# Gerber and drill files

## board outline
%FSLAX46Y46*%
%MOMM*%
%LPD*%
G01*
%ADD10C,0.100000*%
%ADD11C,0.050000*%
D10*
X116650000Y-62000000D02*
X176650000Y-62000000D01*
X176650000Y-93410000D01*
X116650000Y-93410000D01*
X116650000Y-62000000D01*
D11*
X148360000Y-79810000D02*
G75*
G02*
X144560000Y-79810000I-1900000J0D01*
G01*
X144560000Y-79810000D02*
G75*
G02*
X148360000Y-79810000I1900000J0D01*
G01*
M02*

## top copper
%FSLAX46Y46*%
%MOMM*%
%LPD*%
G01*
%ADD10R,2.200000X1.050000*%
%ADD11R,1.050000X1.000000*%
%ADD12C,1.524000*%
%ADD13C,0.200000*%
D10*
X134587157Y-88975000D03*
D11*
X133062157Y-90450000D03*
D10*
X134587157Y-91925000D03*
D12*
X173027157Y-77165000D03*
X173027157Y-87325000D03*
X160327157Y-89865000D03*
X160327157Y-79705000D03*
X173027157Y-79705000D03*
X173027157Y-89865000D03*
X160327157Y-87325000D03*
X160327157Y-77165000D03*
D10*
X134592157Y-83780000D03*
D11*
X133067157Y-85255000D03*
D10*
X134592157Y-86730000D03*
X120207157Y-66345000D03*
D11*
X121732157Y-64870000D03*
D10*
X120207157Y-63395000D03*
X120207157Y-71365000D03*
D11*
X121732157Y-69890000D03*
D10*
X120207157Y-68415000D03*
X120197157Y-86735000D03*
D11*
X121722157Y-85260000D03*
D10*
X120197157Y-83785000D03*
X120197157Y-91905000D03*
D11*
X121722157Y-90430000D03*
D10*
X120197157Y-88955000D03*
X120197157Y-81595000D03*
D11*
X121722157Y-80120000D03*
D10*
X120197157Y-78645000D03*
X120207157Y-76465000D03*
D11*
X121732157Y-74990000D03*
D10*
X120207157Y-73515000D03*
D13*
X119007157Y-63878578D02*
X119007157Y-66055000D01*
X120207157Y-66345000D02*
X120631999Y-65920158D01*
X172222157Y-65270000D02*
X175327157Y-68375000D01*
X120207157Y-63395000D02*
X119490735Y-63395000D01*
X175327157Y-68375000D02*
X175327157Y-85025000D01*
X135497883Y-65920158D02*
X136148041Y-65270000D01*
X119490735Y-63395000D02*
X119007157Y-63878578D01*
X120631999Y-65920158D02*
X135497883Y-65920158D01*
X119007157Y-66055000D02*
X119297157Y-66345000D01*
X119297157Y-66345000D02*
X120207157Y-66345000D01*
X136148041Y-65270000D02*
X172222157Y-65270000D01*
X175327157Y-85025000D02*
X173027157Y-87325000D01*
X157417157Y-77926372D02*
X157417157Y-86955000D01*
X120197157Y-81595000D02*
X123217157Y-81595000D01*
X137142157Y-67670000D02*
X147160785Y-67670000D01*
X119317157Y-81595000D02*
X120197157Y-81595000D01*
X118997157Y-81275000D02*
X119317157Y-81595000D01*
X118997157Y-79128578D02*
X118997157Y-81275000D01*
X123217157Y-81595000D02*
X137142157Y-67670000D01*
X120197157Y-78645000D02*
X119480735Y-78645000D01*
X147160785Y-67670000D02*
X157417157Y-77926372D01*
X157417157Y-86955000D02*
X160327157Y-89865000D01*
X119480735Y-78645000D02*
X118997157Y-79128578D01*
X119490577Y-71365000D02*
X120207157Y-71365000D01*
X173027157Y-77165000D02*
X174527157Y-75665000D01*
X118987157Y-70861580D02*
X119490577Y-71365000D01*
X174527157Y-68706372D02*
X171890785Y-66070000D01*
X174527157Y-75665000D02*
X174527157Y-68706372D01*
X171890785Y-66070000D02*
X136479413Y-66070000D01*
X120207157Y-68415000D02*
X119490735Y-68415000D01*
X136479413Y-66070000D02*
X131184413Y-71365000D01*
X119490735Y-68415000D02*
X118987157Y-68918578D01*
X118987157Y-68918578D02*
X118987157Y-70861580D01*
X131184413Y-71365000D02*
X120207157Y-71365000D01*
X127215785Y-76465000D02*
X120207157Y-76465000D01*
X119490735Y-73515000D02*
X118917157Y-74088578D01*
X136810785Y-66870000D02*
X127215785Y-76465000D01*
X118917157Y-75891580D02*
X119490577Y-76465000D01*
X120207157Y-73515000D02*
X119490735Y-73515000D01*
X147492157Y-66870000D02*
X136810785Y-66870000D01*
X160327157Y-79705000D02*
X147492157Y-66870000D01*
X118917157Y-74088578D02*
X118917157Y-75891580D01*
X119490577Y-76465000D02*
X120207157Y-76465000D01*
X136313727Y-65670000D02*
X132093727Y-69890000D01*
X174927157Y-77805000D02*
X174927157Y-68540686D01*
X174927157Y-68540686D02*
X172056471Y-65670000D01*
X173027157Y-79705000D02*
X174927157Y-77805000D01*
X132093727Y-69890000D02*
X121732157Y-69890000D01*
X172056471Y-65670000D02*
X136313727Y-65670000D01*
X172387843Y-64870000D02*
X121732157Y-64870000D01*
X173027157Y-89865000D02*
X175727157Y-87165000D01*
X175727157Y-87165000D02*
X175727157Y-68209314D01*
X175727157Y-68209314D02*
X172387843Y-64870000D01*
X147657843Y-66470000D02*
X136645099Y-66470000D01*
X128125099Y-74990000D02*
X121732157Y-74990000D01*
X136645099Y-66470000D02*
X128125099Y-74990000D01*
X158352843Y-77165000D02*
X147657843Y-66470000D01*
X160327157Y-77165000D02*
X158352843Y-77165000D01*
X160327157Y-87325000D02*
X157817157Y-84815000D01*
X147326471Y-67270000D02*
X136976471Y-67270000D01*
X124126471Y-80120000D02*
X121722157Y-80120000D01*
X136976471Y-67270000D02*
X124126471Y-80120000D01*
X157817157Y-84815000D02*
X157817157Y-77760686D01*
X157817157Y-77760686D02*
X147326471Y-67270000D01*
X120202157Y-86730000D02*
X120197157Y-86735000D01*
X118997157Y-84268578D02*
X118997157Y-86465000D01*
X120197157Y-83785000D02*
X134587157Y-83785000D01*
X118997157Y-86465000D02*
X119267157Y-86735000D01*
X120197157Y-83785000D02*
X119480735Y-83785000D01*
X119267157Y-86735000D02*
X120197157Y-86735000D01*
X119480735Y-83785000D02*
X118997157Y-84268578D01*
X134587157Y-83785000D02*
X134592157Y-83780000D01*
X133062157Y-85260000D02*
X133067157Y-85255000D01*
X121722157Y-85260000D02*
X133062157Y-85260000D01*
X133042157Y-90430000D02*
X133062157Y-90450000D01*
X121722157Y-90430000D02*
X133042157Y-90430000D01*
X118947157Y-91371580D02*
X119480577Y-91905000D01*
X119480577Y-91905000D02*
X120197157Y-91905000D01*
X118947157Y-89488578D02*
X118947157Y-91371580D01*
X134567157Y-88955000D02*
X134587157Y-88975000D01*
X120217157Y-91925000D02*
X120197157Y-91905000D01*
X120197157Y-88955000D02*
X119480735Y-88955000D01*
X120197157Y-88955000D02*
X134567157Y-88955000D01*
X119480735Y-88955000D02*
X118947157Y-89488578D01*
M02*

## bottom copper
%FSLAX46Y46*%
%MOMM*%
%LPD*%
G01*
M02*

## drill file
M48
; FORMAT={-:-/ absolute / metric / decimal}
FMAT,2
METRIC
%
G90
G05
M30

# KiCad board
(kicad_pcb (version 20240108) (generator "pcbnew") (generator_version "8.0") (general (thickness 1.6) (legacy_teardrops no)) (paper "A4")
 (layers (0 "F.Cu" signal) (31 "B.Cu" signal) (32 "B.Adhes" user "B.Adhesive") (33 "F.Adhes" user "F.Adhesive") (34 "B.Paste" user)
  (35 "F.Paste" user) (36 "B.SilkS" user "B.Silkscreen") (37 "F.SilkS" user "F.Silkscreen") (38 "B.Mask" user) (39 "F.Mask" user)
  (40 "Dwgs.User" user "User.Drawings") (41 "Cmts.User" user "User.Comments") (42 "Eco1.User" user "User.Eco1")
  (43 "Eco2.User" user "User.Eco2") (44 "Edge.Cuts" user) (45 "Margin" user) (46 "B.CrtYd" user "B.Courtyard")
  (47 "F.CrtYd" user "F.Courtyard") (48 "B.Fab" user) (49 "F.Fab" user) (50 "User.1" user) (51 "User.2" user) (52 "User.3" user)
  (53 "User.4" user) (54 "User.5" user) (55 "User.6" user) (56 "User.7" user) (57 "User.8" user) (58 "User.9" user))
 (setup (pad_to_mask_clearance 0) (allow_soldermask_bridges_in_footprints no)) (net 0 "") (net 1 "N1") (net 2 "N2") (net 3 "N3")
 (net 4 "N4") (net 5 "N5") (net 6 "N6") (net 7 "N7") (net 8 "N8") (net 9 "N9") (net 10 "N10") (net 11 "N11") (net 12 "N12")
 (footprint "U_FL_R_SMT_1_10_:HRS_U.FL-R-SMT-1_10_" (layer "F.Cu") (at 134.587157 90.45 -90)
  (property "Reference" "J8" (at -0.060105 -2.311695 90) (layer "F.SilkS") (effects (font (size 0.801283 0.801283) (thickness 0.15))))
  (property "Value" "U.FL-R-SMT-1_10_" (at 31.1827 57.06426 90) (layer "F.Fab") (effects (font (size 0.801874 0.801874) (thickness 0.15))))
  (pad "1" smd rect (at -1.475 0 270) (size 1.05 2.2) (layers "F.Cu" "F.Paste" "F.Mask") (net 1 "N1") (solder_mask_margin 0.102))
  (pad "2" smd rect (at 0 1.525 270) (size 1 1.05) (layers "F.Cu" "F.Paste" "F.Mask") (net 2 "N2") (solder_mask_margin 0.102))
  (pad "3" smd rect (at 1.475 0 270) (size 1.05 2.2) (layers "F.Cu" "F.Paste" "F.Mask") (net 1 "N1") (solder_mask_margin 0.102))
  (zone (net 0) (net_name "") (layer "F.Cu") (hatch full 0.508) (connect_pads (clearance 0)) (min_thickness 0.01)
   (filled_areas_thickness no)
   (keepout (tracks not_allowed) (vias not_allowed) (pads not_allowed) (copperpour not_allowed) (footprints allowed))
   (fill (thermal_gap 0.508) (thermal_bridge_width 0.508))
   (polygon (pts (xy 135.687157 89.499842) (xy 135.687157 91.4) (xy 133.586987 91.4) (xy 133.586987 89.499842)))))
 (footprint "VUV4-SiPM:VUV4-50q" (layer "F.Cu") (at 166.677157 83.515)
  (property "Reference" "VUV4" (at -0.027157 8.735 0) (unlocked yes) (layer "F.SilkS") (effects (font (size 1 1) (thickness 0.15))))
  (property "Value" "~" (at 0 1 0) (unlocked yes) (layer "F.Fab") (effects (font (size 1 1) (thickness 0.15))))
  (pad "1" smd circle (at 6.35 -6.35 90) (size 1.524 1.524) (layers "F.Cu" "F.Paste" "F.Mask") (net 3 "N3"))
  (pad "2" smd circle (at 6.35 3.81) (size 1.524 1.524) (layers "F.Cu" "F.Paste" "F.Mask") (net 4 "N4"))
  (pad "3" smd circle (at -6.35 6.35) (size 1.524 1.524) (layers "F.Cu" "F.Paste" "F.Mask") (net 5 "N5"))
  (pad "4" smd circle (at -6.35 -3.81) (size 1.524 1.524) (layers "F.Cu" "F.Paste" "F.Mask") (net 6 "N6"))
  (pad "5" smd circle (at 6.35 -3.81) (size 1.524 1.524) (layers "F.Cu" "F.Paste" "F.Mask") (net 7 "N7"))
  (pad "6" smd circle (at 6.35 6.35) (size 1.524 1.524) (layers "F.Cu" "F.Paste" "F.Mask") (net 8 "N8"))
  (pad "7" smd circle (at -6.35 3.81) (size 1.524 1.524) (layers "F.Cu" "F.Paste" "F.Mask") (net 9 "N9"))
  (pad "8" smd circle (at -6.35 -6.35) (size 1.524 1.524) (layers "F.Cu" "F.Paste" "F.Mask") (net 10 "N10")))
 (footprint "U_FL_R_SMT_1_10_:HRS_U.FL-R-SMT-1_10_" (layer "F.Cu") (at 134.592157 85.255 -90)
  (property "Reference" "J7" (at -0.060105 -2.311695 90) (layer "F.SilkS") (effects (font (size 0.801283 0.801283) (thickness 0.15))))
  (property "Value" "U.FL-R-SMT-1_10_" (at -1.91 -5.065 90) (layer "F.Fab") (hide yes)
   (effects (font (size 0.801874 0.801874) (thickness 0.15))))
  (pad "1" smd rect (at -1.475 0 270) (size 1.05 2.2) (layers "F.Cu" "F.Paste" "F.Mask") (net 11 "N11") (solder_mask_margin 0.102))
  (pad "2" smd rect (at 0 1.525 270) (size 1 1.05) (layers "F.Cu" "F.Paste" "F.Mask") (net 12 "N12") (solder_mask_margin 0.102))
  (pad "3" smd rect (at 1.475 0 270) (size 1.05 2.2) (layers "F.Cu" "F.Paste" "F.Mask") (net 11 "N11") (solder_mask_margin 0.102))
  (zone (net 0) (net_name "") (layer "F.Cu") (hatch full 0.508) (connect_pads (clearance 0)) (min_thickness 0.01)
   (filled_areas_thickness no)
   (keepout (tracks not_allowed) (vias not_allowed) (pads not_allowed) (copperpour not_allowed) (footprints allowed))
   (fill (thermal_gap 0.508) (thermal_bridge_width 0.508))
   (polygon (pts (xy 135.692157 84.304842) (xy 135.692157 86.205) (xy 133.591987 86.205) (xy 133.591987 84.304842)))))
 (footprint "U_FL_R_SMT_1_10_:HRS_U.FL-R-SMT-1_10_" (layer "F.Cu") (at 120.207157 64.87 90)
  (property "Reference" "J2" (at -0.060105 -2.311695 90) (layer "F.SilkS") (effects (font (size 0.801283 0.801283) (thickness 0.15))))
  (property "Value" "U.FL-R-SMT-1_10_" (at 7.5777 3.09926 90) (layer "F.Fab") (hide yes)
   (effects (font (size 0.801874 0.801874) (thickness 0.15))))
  (pad "1" smd rect (at -1.475 0 90) (size 1.05 2.2) (layers "F.Cu" "F.Paste" "F.Mask") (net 4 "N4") (solder_mask_margin 0.102))
  (pad "2" smd rect (at 0 1.525 90) (size 1 1.05) (layers "F.Cu" "F.Paste" "F.Mask") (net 8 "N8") (solder_mask_margin 0.102))
  (pad "3" smd rect (at 1.475 0 90) (size 1.05 2.2) (layers "F.Cu" "F.Paste" "F.Mask") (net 4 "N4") (solder_mask_margin 0.102))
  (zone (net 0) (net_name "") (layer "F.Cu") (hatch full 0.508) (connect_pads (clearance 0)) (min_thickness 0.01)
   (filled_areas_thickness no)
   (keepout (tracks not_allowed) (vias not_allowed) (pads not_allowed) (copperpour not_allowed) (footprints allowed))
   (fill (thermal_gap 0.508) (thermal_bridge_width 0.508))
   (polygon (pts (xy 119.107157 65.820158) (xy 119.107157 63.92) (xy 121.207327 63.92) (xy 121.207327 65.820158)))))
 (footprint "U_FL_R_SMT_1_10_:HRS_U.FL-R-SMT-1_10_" (layer "F.Cu") (at 120.207157 69.89 90)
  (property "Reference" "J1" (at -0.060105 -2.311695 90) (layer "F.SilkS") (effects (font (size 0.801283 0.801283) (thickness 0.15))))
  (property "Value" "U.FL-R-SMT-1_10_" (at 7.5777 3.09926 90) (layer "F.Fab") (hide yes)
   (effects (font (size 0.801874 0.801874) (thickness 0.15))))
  (pad "1" smd rect (at -1.475 0 90) (size 1.05 2.2) (layers "F.Cu" "F.Paste" "F.Mask") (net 3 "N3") (solder_mask_margin 0.102))
  (pad "2" smd rect (at 0 1.525 90) (size 1 1.05) (layers "F.Cu" "F.Paste" "F.Mask") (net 7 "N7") (solder_mask_margin 0.102))
  (pad "3" smd rect (at 1.475 0 90) (size 1.05 2.2) (layers "F.Cu" "F.Paste" "F.Mask") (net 3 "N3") (solder_mask_margin 0.102))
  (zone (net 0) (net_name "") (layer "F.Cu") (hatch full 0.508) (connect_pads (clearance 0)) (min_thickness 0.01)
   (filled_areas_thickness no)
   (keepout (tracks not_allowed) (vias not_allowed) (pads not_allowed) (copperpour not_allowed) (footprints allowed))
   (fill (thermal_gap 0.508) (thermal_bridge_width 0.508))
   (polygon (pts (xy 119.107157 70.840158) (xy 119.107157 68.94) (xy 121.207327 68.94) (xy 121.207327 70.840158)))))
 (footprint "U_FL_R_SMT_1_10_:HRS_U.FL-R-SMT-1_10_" (layer "F.Cu") (at 120.197157 85.26 90)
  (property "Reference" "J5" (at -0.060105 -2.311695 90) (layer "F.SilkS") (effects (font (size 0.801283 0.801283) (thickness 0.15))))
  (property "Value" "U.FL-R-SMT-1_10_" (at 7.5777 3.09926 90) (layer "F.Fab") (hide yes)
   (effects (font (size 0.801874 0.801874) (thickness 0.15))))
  (pad "1" smd rect (at -1.475 0 90) (size 1.05 2.2) (layers "F.Cu" "F.Paste" "F.Mask") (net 11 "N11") (solder_mask_margin 0.102))
  (pad "2" smd rect (at 0 1.525 90) (size 1 1.05) (layers "F.Cu" "F.Paste" "F.Mask") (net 12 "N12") (solder_mask_margin 0.102))
  (pad "3" smd rect (at 1.475 0 90) (size 1.05 2.2) (layers "F.Cu" "F.Paste" "F.Mask") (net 11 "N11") (solder_mask_margin 0.102))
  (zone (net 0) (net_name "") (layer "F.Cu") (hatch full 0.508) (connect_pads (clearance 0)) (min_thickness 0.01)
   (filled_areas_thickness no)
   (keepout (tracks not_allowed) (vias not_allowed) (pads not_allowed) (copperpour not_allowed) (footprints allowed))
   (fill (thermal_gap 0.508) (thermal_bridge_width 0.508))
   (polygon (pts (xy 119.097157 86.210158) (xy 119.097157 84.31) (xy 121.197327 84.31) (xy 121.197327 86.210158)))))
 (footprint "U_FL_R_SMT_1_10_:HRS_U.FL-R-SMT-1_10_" (layer "F.Cu") (at 120.197157 90.43 90)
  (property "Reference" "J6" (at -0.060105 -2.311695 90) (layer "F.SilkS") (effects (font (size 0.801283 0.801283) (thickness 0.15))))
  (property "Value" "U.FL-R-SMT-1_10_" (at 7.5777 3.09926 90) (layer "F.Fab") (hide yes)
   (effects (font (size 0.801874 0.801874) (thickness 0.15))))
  (pad "1" smd rect (at -1.475 0 90) (size 1.05 2.2) (layers "F.Cu" "F.Paste" "F.Mask") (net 1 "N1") (solder_mask_margin 0.102))
  (pad "2" smd rect (at 0 1.525 90) (size 1 1.05) (layers "F.Cu" "F.Paste" "F.Mask") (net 2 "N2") (solder_mask_margin 0.102))
  (pad "3" smd rect (at 1.475 0 90) (size 1.05 2.2) (layers "F.Cu" "F.Paste" "F.Mask") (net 1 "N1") (solder_mask_margin 0.102))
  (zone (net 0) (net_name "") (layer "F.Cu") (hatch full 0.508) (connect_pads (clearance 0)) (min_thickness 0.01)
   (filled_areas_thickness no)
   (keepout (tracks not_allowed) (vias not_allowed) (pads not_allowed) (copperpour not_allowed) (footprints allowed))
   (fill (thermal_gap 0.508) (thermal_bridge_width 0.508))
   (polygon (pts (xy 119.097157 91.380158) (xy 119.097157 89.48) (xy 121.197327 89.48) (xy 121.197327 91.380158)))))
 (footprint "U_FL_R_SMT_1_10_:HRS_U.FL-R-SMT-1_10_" (layer "F.Cu") (at 120.197157 80.12 90)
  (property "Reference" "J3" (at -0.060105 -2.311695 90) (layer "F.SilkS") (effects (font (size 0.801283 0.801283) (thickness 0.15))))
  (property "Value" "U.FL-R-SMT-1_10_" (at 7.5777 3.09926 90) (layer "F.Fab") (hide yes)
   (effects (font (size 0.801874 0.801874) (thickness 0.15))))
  (pad "1" smd rect (at -1.475 0 90) (size 1.05 2.2) (layers "F.Cu" "F.Paste" "F.Mask") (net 5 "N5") (solder_mask_margin 0.102))
  (pad "2" smd rect (at 0 1.525 90) (size 1 1.05) (layers "F.Cu" "F.Paste" "F.Mask") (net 9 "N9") (solder_mask_margin 0.102))
  (pad "3" smd rect (at 1.475 0 90) (size 1.05 2.2) (layers "F.Cu" "F.Paste" "F.Mask") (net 5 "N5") (solder_mask_margin 0.102))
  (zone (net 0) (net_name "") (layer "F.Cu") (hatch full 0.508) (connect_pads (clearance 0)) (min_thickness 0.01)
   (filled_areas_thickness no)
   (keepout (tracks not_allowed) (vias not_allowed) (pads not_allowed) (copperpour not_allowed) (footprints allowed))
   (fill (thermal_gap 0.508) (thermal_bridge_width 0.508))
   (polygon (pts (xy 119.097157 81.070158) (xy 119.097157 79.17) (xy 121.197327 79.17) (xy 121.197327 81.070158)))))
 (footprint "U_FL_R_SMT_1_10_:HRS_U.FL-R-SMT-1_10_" (layer "F.Cu") (at 120.207157 74.99 90)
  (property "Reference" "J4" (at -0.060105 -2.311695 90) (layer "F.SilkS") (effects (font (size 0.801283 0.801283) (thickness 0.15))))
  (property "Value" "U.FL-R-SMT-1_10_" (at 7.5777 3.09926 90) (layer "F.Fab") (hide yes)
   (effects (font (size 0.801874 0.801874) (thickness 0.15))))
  (pad "1" smd rect (at -1.475 0 90) (size 1.05 2.2) (layers "F.Cu" "F.Paste" "F.Mask") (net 6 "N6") (solder_mask_margin 0.102))
  (pad "2" smd rect (at 0 1.525 90) (size 1 1.05) (layers "F.Cu" "F.Paste" "F.Mask") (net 10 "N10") (solder_mask_margin 0.102))
  (pad "3" smd rect (at 1.475 0 90) (size 1.05 2.2) (layers "F.Cu" "F.Paste" "F.Mask") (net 6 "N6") (solder_mask_margin 0.102))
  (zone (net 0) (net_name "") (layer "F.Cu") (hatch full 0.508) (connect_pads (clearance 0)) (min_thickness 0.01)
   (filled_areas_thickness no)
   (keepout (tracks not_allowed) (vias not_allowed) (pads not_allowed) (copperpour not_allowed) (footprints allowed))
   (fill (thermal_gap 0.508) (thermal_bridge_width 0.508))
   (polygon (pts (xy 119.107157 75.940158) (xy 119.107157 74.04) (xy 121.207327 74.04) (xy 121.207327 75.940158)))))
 (gr_rect (start 116.65 62) (end 176.65 93.41) (stroke (width 0.1) (type default)) (fill none) (layer "Edge.Cuts"))
 (gr_circle (center 146.46 79.81) (end 148.36 79.81) (stroke (width 0.05) (type default)) (fill none) (layer "Edge.Cuts"))
 (segment (start 119.007157 63.878578) (end 119.007157 66.055) (width 0.2) (layer "F.Cu") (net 4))
 (segment (start 120.207157 66.345) (end 120.631999 65.920158) (width 0.2) (layer "F.Cu") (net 4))
 (segment (start 172.222157 65.27) (end 175.327157 68.375) (width 0.2) (layer "F.Cu") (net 4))
 (segment (start 120.207157 63.395) (end 119.490735 63.395) (width 0.2) (layer "F.Cu") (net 4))
 (segment (start 175.327157 68.375) (end 175.327157 85.025) (width 0.2) (layer "F.Cu") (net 4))
 (segment (start 135.497883 65.920158) (end 136.148041 65.27) (width 0.2) (layer "F.Cu") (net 4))
 (segment (start 119.490735 63.395) (end 119.007157 63.878578) (width 0.2) (layer "F.Cu") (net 4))
 (segment (start 120.631999 65.920158) (end 135.497883 65.920158) (width 0.2) (layer "F.Cu") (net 4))
 (segment (start 119.007157 66.055) (end 119.297157 66.345) (width 0.2) (layer "F.Cu") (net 4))
 (segment (start 119.297157 66.345) (end 120.207157 66.345) (width 0.2) (layer "F.Cu") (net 4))
 (segment (start 136.148041 65.27) (end 172.222157 65.27) (width 0.2) (layer "F.Cu") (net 4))
 (segment (start 175.327157 85.025) (end 173.027157 87.325) (width 0.2) (layer "F.Cu") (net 4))
 (segment (start 157.417157 77.926372) (end 157.417157 86.955) (width 0.2) (layer "F.Cu") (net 5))
 (segment (start 120.197157 81.595) (end 123.217157 81.595) (width 0.2) (layer "F.Cu") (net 5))
 (segment (start 137.142157 67.67) (end 147.160785 67.67) (width 0.2) (layer "F.Cu") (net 5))
 (segment (start 119.317157 81.595) (end 120.197157 81.595) (width 0.2) (layer "F.Cu") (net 5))
 (segment (start 118.997157 81.275) (end 119.317157 81.595) (width 0.2) (layer "F.Cu") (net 5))
 (segment (start 118.997157 79.128578) (end 118.997157 81.275) (width 0.2) (layer "F.Cu") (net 5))
 (segment (start 123.217157 81.595) (end 137.142157 67.67) (width 0.2) (layer "F.Cu") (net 5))
 (segment (start 120.197157 78.645) (end 119.480735 78.645) (width 0.2) (layer "F.Cu") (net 5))
 (segment (start 147.160785 67.67) (end 157.417157 77.926372) (width 0.2) (layer "F.Cu") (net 5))
 (segment (start 157.417157 86.955) (end 160.327157 89.865) (width 0.2) (layer "F.Cu") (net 5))
 (segment (start 119.480735 78.645) (end 118.997157 79.128578) (width 0.2) (layer "F.Cu") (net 5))
 (segment (start 119.490577 71.365) (end 120.207157 71.365) (width 0.2) (layer "F.Cu") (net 3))
 (segment (start 173.027157 77.165) (end 174.527157 75.665) (width 0.2) (layer "F.Cu") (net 3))
 (segment (start 118.987157 70.86158) (end 119.490577 71.365) (width 0.2) (layer "F.Cu") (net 3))
 (segment (start 174.527157 68.706372) (end 171.890785 66.07) (width 0.2) (layer "F.Cu") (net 3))
 (segment (start 174.527157 75.665) (end 174.527157 68.706372) (width 0.2) (layer "F.Cu") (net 3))
 (segment (start 171.890785 66.07) (end 136.479413 66.07) (width 0.2) (layer "F.Cu") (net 3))
 (segment (start 120.207157 68.415) (end 119.490735 68.415) (width 0.2) (layer "F.Cu") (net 3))
 (segment (start 136.479413 66.07) (end 131.184413 71.365) (width 0.2) (layer "F.Cu") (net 3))
 (segment (start 119.490735 68.415) (end 118.987157 68.918578) (width 0.2) (layer "F.Cu") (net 3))
 (segment (start 118.987157 68.918578) (end 118.987157 70.86158) (width 0.2) (layer "F.Cu") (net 3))
 (segment (start 131.184413 71.365) (end 120.207157 71.365) (width 0.2) (layer "F.Cu") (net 3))
 (segment (start 127.215785 76.465) (end 120.207157 76.465) (width 0.2) (layer "F.Cu") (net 6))
 (segment (start 119.490735 73.515) (end 118.917157 74.088578) (width 0.2) (layer "F.Cu") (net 6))
 (segment (start 136.810785 66.87) (end 127.215785 76.465) (width 0.2) (layer "F.Cu") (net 6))
 (segment (start 118.917157 75.89158) (end 119.490577 76.465) (width 0.2) (layer "F.Cu") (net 6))
 (segment (start 120.207157 73.515) (end 119.490735 73.515) (width 0.2) (layer "F.Cu") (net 6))
 (segment (start 147.492157 66.87) (end 136.810785 66.87) (width 0.2) (layer "F.Cu") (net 6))
 (segment (start 160.327157 79.705) (end 147.492157 66.87) (width 0.2) (layer "F.Cu") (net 6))
 (segment (start 118.917157 74.088578) (end 118.917157 75.89158) (width 0.2) (layer "F.Cu") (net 6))
 (segment (start 119.490577 76.465) (end 120.207157 76.465) (width 0.2) (layer "F.Cu") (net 6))
 (segment (start 136.313727 65.67) (end 132.093727 69.89) (width 0.2) (layer "F.Cu") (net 7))
 (segment (start 174.927157 77.805) (end 174.927157 68.540686) (width 0.2) (layer "F.Cu") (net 7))
 (segment (start 174.927157 68.540686) (end 172.056471 65.67) (width 0.2) (layer "F.Cu") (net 7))
 (segment (start 173.027157 79.705) (end 174.927157 77.805) (width 0.2) (layer "F.Cu") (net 7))
 (segment (start 132.093727 69.89) (end 121.732157 69.89) (width 0.2) (layer "F.Cu") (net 7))
 (segment (start 172.056471 65.67) (end 136.313727 65.67) (width 0.2) (layer "F.Cu") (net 7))
 (segment (start 172.387843 64.87) (end 121.732157 64.87) (width 0.2) (layer "F.Cu") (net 8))
 (segment (start 173.027157 89.865) (end 175.727157 87.165) (width 0.2) (layer "F.Cu") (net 8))
 (segment (start 175.727157 87.165) (end 175.727157 68.209314) (width 0.2) (layer "F.Cu") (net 8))
 (segment (start 175.727157 68.209314) (end 172.387843 64.87) (width 0.2) (layer "F.Cu") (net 8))
 (segment (start 147.657843 66.47) (end 136.645099 66.47) (width 0.2) (layer "F.Cu") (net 10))
 (segment (start 128.125099 74.99) (end 121.732157 74.99) (width 0.2) (layer "F.Cu") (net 10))
 (segment (start 136.645099 66.47) (end 128.125099 74.99) (width 0.2) (layer "F.Cu") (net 10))
 (segment (start 158.352843 77.165) (end 147.657843 66.47) (width 0.2) (layer "F.Cu") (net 10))
 (segment (start 160.327157 77.165) (end 158.352843 77.165) (width 0.2) (layer "F.Cu") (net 10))
 (segment (start 160.327157 87.325) (end 157.817157 84.815) (width 0.2) (layer "F.Cu") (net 9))
 (segment (start 147.326471 67.27) (end 136.976471 67.27) (width 0.2) (layer "F.Cu") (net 9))
 (segment (start 124.126471 80.12) (end 121.722157 80.12) (width 0.2) (layer "F.Cu") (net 9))
 (segment (start 136.976471 67.27) (end 124.126471 80.12) (width 0.2) (layer "F.Cu") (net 9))
 (segment (start 157.817157 84.815) (end 157.817157 77.760686) (width 0.2) (layer "F.Cu") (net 9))
 (segment (start 157.817157 77.760686) (end 147.326471 67.27) (width 0.2) (layer "F.Cu") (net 9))
 (segment (start 120.202157 86.73) (end 120.197157 86.735) (width 0.2) (layer "F.Cu") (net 11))
 (segment (start 118.997157 84.268578) (end 118.997157 86.465) (width 0.2) (layer "F.Cu") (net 11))
 (segment (start 120.197157 83.785) (end 134.587157 83.785) (width 0.2) (layer "F.Cu") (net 11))
 (segment (start 118.997157 86.465) (end 119.267157 86.735) (width 0.2) (layer "F.Cu") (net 11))
 (segment (start 120.197157 83.785) (end 119.480735 83.785) (width 0.2) (layer "F.Cu") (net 11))
 (segment (start 119.267157 86.735) (end 120.197157 86.735) (width 0.2) (layer "F.Cu") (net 11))
 (segment (start 119.480735 83.785) (end 118.997157 84.268578) (width 0.2) (layer "F.Cu") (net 11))
 (segment (start 134.587157 83.785) (end 134.592157 83.78) (width 0.2) (layer "F.Cu") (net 11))
 (segment (start 133.062157 85.26) (end 133.067157 85.255) (width 0.2) (layer "F.Cu") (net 12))
 (segment (start 121.722157 85.26) (end 133.062157 85.26) (width 0.2) (layer "F.Cu") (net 12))
 (segment (start 133.042157 90.43) (end 133.062157 90.45) (width 0.2) (layer "F.Cu") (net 2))
 (segment (start 121.722157 90.43) (end 133.042157 90.43) (width 0.2) (layer "F.Cu") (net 2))
 (segment (start 118.947157 91.37158) (end 119.480577 91.905) (width 0.2) (layer "F.Cu") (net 1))
 (segment (start 119.480577 91.905) (end 120.197157 91.905) (width 0.2) (layer "F.Cu") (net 1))
 (segment (start 118.947157 89.488578) (end 118.947157 91.37158) (width 0.2) (layer "F.Cu") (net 1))
 (segment (start 134.567157 88.955) (end 134.587157 88.975) (width 0.2) (layer "F.Cu") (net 1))
 (segment (start 120.217157 91.925) (end 120.197157 91.905) (width 0.2) (layer "F.Cu") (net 1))
 (segment (start 120.197157 88.955) (end 119.480735 88.955) (width 0.2) (layer "F.Cu") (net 1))
 (segment (start 120.197157 88.955) (end 134.567157 88.955) (width 0.2) (layer "F.Cu") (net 1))
 (segment (start 119.480735 88.955) (end 118.947157 89.488578) (width 0.2) (layer "F.Cu") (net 1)))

